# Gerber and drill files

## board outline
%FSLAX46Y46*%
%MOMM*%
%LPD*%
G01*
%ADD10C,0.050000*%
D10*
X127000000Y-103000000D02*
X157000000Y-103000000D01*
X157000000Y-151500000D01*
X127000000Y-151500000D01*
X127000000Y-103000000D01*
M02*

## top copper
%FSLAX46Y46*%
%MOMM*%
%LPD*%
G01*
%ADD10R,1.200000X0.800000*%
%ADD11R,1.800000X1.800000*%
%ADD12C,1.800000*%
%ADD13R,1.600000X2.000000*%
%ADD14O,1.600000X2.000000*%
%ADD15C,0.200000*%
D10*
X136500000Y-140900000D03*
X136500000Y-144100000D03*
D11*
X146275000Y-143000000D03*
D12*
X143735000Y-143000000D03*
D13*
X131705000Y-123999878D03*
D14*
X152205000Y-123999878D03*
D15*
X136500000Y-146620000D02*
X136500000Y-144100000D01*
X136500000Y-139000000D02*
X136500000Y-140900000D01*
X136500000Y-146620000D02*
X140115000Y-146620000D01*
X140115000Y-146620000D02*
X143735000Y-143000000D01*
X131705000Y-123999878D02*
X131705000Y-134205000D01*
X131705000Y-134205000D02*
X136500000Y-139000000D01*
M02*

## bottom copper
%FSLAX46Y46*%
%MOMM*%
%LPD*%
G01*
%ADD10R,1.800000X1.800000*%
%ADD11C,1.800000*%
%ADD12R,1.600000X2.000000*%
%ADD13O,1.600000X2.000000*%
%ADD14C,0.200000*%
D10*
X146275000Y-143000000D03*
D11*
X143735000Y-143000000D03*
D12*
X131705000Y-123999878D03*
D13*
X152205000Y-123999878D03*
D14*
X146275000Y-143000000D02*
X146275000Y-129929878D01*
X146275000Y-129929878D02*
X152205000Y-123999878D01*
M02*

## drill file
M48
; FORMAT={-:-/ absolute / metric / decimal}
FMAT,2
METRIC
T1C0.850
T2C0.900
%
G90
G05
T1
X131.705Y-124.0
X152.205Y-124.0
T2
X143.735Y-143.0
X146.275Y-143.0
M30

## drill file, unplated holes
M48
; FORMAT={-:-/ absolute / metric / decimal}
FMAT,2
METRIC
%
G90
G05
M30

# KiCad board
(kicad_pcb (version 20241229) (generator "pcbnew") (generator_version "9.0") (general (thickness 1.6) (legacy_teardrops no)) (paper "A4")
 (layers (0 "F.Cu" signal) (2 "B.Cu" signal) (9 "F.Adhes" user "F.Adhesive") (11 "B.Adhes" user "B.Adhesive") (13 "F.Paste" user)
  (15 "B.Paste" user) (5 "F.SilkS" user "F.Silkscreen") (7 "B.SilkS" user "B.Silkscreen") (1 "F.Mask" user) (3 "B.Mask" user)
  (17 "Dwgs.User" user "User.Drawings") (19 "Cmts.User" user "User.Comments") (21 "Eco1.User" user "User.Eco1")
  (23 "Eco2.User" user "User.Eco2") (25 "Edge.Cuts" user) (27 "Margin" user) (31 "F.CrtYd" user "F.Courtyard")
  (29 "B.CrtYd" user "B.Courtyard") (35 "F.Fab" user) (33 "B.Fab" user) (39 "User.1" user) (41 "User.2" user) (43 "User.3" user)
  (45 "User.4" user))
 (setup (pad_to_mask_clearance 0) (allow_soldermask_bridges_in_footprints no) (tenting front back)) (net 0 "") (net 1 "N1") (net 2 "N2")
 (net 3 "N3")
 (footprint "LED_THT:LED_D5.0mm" (layer "F.Cu") (at 146.275 143 180)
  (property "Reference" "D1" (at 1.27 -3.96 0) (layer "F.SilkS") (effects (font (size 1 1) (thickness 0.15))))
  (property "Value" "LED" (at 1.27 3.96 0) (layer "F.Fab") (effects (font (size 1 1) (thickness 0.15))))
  (pad "1" thru_hole rect (at 0 0 180) (size 1.8 1.8) (drill 0.9) (layers "*.Cu" "*.Mask") (remove_unused_layers no) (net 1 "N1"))
  (pad "2" thru_hole circle (at 2.54 0 180) (size 1.8 1.8) (drill 0.9) (layers "*.Cu" "*.Mask") (remove_unused_layers no) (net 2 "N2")))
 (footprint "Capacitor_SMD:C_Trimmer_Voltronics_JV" (layer "F.Cu") (at 136.5 142.5 -90)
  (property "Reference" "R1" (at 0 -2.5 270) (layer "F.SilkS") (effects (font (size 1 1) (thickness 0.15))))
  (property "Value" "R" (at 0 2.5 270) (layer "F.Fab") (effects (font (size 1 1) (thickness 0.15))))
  (pad "1" smd rect (at -1.6 0 270) (size 0.8 1.2) (layers "F.Cu" "F.Mask" "F.Paste") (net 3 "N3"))
  (pad "2" smd rect (at 1.6 0 270) (size 0.8 1.2) (layers "F.Cu" "F.Mask" "F.Paste") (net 2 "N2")))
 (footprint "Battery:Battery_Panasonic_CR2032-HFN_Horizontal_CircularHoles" (layer "F.Cu") (at 131.705 123.999878)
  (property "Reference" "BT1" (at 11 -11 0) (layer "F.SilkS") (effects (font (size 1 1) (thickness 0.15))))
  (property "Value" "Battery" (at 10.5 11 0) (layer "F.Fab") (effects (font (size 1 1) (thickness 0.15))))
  (pad "1" thru_hole rect (at 0 0) (size 1.6 2) (drill 0.85) (layers "*.Cu" "*.Mask") (remove_unused_layers no) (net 3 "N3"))
  (pad "2" thru_hole oval (at 20.5 0) (size 1.6 2) (drill 0.85) (layers "*.Cu" "*.Mask") (remove_unused_layers no) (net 1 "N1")))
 (gr_rect (start 127 103) (end 157 151.5) (stroke (width 0.05) (type default)) (fill no) (layer "Edge.Cuts"))
 (segment (start 146.275 129.929878) (end 152.205 123.999878) (width 0.2) (layer "B.Cu") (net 1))
 (segment (start 146.275 143) (end 146.275 129.929878) (width 0.2) (layer "B.Cu") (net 1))
 (segment (start 131.705 123.999878) (end 131.705 134.205) (width 0.2) (layer "F.Cu") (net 3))
 (segment (start 131.705 134.205) (end 136.5 139) (width 0.2) (layer "F.Cu") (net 3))
 (segment (start 136.5 139) (end 136.5 140.9) (width 0.2) (layer "F.Cu") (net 3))
 (segment (start 136.5 146.62) (end 136.5 144.1) (width 0.2) (layer "F.Cu") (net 2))
 (segment (start 140.115 146.62) (end 143.735 143) (width 0.2) (layer "F.Cu") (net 2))
 (segment (start 136.5 146.62) (end 140.115 146.62) (width 0.2) (layer "F.Cu") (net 2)))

